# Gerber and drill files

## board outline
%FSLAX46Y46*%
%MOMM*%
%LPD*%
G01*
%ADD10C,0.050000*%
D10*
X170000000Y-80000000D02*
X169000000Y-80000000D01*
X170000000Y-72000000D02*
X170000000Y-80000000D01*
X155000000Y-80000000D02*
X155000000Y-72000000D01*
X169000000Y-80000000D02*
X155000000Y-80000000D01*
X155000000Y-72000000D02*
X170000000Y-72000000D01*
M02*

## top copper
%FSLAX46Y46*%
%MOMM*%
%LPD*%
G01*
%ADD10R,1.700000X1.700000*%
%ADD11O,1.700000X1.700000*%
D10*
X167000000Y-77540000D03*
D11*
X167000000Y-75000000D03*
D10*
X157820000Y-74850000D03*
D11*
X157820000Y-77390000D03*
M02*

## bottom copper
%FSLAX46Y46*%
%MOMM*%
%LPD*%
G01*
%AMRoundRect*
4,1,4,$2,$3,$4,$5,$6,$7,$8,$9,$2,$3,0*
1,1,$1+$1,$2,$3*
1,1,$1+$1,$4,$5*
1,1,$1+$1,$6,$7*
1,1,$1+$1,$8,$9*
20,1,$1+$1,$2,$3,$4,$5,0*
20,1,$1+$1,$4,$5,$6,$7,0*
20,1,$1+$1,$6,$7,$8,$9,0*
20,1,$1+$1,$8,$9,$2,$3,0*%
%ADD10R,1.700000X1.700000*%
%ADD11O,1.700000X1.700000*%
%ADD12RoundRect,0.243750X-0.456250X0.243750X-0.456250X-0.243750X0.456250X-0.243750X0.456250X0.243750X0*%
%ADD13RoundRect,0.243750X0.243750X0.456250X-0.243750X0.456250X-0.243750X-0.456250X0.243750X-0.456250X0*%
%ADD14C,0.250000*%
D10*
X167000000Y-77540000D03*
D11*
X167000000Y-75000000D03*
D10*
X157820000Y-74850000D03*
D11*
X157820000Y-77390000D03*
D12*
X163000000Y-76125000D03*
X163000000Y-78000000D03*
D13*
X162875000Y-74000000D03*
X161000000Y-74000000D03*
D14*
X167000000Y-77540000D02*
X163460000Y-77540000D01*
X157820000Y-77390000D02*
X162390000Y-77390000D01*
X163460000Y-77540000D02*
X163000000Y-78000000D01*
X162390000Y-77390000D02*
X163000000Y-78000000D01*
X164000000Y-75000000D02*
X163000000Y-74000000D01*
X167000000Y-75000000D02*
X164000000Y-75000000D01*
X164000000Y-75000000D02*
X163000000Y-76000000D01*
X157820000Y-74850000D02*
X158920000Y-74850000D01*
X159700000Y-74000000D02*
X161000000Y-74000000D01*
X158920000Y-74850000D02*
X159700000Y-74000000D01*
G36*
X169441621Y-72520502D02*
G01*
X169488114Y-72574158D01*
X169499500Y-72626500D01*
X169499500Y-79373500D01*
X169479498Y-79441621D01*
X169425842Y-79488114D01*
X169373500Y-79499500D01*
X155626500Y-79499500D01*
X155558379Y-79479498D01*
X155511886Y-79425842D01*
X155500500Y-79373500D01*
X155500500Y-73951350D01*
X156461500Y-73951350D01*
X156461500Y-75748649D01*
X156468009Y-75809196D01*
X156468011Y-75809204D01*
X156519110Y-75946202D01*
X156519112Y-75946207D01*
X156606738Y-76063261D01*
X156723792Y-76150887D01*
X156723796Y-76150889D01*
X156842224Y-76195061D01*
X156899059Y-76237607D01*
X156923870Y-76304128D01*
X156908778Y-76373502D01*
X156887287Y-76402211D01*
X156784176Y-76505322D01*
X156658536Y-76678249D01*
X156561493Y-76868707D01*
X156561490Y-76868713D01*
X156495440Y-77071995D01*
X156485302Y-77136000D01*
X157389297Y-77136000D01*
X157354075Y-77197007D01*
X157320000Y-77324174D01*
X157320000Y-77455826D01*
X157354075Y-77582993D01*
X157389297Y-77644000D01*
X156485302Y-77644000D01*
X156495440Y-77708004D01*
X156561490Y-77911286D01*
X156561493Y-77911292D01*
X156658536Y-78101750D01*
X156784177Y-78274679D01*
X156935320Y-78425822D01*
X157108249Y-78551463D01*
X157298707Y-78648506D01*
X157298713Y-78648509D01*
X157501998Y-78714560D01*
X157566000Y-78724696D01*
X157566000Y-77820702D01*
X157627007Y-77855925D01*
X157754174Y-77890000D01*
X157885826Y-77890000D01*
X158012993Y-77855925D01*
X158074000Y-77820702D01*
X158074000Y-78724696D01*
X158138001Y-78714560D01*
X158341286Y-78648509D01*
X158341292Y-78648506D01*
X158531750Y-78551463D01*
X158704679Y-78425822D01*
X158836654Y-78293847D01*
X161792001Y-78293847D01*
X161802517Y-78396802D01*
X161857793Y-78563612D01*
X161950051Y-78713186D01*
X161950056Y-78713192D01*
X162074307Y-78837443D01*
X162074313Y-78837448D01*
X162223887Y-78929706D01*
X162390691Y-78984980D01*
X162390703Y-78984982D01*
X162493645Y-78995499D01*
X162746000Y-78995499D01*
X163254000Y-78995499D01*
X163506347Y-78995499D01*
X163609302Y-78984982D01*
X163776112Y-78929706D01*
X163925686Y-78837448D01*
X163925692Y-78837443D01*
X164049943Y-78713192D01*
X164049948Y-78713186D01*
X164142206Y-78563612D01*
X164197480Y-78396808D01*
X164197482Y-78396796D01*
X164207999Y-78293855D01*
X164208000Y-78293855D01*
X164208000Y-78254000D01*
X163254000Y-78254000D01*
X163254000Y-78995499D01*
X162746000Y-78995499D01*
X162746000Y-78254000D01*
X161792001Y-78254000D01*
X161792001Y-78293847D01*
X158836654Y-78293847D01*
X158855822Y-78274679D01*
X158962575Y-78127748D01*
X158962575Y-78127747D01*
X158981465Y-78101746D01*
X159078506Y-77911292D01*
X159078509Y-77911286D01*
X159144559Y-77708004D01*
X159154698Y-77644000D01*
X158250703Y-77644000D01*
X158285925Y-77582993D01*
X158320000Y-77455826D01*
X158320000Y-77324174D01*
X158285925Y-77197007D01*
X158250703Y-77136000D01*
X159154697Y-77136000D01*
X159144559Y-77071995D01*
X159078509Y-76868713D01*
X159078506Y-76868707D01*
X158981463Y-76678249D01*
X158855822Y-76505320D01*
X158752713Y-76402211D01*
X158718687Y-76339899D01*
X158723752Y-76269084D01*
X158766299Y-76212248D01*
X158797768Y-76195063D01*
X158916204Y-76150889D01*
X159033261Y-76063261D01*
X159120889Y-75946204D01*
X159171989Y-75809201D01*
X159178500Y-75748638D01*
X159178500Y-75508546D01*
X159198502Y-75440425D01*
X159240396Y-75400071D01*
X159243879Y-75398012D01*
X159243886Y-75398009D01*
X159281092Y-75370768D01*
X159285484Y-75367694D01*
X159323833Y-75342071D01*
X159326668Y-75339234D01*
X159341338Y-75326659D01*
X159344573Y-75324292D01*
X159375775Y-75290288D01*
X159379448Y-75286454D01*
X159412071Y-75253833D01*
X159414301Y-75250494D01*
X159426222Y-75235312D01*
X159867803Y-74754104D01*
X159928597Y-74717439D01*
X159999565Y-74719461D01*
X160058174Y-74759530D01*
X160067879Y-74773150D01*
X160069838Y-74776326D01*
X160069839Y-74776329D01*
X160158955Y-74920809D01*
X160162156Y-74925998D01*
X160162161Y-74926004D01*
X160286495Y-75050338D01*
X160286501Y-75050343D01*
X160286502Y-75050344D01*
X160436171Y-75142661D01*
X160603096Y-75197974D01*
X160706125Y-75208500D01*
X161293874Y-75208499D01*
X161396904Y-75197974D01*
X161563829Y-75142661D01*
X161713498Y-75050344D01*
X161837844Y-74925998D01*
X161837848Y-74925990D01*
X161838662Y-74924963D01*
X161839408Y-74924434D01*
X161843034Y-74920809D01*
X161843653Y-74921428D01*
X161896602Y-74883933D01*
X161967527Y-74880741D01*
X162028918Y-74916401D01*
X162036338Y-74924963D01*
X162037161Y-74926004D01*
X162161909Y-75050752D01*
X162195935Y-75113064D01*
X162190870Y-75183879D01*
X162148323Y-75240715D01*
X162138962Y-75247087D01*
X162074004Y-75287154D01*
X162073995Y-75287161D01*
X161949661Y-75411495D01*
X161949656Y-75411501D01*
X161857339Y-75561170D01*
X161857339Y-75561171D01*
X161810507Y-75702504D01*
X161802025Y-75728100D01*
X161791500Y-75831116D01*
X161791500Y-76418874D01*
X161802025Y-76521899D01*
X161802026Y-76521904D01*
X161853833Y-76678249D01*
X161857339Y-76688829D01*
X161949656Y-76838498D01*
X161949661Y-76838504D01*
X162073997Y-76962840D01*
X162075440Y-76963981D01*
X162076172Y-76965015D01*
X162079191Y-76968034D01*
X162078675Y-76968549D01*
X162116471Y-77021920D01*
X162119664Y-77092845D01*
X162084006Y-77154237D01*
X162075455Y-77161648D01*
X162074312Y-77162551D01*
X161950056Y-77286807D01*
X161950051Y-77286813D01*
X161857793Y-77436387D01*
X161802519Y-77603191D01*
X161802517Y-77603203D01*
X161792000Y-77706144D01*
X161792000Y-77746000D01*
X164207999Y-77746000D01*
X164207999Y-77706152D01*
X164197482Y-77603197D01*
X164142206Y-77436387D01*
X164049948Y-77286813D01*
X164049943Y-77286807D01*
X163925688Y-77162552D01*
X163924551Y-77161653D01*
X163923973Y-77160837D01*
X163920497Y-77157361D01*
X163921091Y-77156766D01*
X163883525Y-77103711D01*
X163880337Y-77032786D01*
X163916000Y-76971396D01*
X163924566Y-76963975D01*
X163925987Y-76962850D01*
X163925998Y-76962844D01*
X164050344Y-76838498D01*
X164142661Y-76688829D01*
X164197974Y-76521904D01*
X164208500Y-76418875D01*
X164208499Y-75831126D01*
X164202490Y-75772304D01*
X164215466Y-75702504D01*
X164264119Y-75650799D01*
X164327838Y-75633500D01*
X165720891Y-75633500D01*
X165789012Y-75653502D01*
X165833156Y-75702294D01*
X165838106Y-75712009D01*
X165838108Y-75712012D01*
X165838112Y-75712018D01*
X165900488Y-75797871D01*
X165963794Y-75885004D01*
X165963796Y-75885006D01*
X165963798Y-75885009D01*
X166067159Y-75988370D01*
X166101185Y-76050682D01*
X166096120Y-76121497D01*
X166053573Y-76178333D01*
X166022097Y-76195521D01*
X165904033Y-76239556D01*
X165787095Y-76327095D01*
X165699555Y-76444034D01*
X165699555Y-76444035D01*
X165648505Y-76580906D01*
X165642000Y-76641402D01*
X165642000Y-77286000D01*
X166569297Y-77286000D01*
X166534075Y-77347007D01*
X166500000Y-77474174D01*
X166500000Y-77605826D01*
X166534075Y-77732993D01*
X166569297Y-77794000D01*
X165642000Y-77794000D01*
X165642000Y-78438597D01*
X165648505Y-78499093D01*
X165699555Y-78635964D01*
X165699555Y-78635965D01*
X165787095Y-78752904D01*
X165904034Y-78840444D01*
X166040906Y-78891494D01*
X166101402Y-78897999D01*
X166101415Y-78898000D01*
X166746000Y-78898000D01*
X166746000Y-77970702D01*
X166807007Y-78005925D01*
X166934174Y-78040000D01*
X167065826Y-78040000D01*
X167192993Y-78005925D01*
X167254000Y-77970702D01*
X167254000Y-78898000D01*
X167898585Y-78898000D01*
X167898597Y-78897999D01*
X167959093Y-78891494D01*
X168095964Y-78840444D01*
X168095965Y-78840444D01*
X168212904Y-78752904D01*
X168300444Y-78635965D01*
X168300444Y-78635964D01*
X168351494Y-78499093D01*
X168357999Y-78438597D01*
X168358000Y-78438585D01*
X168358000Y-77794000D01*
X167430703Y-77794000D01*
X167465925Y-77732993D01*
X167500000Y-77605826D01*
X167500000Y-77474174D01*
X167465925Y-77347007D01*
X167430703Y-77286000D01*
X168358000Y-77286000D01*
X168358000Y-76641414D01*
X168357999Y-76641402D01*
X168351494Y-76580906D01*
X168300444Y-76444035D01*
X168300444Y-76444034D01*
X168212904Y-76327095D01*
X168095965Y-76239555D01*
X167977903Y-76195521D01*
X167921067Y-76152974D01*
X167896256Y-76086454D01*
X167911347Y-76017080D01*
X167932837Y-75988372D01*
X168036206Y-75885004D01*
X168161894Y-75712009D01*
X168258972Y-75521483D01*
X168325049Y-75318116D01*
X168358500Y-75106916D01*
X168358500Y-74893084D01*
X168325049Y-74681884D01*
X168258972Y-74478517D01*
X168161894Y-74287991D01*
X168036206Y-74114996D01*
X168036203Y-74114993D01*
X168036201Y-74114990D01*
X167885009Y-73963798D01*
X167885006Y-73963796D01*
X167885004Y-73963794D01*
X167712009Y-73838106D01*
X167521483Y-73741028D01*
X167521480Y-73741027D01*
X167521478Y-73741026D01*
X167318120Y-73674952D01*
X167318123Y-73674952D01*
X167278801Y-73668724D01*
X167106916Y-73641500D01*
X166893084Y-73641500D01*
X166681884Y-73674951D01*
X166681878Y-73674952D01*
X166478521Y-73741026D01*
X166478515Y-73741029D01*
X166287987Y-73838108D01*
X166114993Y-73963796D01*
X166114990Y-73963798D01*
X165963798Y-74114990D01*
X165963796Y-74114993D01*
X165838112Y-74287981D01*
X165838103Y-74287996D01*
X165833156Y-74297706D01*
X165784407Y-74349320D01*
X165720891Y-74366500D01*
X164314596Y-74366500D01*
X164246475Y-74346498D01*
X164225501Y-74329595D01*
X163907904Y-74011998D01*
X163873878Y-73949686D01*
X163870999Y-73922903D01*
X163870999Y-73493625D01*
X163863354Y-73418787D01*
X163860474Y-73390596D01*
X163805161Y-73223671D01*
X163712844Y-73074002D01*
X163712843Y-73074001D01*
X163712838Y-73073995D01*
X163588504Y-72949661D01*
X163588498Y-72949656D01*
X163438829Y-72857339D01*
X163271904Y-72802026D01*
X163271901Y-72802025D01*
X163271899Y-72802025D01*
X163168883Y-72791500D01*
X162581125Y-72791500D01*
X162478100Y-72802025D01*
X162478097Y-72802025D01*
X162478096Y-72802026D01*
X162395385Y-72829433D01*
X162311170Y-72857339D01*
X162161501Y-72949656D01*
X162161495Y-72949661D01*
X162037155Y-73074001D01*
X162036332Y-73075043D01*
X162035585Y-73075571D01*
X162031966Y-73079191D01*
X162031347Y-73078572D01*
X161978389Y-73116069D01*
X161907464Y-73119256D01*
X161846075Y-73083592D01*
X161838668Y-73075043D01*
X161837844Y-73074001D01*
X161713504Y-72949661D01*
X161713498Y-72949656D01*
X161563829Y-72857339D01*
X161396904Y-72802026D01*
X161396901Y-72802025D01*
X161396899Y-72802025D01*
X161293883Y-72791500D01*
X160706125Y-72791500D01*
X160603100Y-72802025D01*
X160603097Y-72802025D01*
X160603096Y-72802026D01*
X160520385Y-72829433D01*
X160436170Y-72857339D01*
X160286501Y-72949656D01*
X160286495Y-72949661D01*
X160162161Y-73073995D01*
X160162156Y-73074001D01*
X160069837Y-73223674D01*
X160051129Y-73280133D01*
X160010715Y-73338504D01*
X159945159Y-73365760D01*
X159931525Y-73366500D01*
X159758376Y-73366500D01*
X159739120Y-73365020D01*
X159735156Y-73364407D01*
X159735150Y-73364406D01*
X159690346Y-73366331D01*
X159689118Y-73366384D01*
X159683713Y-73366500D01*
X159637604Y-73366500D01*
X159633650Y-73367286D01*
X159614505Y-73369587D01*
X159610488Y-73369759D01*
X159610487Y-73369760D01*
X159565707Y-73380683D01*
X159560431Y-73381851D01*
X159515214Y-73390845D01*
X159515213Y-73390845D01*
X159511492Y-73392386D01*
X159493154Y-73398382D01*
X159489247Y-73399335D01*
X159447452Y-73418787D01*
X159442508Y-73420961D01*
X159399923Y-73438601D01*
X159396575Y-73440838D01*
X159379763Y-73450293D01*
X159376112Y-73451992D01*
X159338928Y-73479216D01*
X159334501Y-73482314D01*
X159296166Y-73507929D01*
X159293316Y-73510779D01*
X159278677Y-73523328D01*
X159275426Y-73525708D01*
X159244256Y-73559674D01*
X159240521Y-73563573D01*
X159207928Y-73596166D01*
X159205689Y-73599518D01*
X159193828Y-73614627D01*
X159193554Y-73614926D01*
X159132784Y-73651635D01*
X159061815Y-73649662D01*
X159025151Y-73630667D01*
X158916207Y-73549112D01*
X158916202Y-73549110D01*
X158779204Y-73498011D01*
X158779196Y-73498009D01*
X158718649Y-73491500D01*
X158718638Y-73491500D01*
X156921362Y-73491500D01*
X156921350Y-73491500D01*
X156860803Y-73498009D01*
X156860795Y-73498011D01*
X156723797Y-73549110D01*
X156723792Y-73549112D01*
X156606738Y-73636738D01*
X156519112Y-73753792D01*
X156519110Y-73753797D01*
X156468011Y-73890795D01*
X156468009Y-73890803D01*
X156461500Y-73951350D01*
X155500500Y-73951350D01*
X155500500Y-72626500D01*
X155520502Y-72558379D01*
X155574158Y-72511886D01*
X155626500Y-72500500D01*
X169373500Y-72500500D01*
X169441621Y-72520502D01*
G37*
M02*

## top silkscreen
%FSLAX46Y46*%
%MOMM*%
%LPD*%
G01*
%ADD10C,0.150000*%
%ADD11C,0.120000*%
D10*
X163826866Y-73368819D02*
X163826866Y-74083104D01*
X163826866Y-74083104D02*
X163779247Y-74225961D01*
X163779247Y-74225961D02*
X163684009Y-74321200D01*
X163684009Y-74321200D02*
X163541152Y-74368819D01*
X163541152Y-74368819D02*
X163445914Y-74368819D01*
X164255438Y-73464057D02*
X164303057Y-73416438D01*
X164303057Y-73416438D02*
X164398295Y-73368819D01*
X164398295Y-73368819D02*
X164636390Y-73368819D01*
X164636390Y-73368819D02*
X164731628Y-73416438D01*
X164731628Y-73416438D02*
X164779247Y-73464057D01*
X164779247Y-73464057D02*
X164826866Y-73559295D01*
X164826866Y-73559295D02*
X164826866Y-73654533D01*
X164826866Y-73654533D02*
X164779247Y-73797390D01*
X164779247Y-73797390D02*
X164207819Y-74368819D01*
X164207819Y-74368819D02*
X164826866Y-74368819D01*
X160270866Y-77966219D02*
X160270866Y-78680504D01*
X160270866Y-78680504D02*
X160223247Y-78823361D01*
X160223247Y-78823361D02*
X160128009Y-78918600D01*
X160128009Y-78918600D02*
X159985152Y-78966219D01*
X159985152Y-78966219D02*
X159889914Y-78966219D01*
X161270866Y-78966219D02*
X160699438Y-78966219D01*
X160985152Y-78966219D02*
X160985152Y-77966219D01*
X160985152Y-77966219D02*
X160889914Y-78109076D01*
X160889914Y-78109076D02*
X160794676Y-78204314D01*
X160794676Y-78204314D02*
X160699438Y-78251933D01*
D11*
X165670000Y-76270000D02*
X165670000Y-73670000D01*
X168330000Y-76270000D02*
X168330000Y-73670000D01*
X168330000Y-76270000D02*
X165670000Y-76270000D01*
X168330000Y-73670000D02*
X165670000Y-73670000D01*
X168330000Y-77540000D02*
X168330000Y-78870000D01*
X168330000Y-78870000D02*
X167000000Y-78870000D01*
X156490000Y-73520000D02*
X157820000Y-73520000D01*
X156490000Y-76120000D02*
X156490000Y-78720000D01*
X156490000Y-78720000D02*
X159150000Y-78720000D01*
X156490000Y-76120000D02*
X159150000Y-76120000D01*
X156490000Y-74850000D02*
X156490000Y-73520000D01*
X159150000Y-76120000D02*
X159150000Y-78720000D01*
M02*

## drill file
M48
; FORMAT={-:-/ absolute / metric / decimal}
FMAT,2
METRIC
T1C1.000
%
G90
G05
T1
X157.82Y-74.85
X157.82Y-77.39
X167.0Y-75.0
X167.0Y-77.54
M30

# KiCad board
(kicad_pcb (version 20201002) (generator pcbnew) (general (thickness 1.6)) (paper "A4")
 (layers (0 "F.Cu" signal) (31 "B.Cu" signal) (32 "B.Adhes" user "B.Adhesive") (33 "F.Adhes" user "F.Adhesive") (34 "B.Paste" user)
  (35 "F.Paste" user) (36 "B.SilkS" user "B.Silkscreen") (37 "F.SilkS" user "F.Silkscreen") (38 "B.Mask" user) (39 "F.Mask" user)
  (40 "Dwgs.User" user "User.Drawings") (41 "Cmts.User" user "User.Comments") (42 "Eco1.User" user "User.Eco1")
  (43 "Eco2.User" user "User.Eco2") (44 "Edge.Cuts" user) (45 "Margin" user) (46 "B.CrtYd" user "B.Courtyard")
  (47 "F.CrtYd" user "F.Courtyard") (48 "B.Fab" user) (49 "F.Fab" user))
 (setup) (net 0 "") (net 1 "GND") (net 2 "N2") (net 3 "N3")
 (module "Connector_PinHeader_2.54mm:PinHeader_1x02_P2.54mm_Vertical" (layer "F.Cu") (at 167 77.54 180)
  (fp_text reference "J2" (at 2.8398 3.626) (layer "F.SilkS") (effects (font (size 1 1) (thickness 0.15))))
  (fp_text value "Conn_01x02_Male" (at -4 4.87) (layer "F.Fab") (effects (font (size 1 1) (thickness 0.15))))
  (fp_line (start 1.33 1.27) (end 1.33 3.87) (layer "F.SilkS") (width 0.12))
  (fp_line (start -1.33 1.27) (end -1.33 3.87) (layer "F.SilkS") (width 0.12))
  (fp_line (start -1.33 1.27) (end 1.33 1.27) (layer "F.SilkS") (width 0.12))
  (fp_line (start -1.33 3.87) (end 1.33 3.87) (layer "F.SilkS") (width 0.12))
  (fp_line (start -1.33 0) (end -1.33 -1.33) (layer "F.SilkS") (width 0.12))
  (fp_line (start -1.33 -1.33) (end 0 -1.33) (layer "F.SilkS") (width 0.12))
  (pad "1" thru_hole rect (at 0 0 180) (size 1.7 1.7) (drill 1) (layers *.Cu *.Mask) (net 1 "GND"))
  (pad "2" thru_hole oval (at 0 2.54 180) (size 1.7 1.7) (drill 1) (layers *.Cu *.Mask) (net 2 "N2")))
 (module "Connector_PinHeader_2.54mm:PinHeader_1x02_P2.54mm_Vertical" (layer "F.Cu") (at 157.82 74.85)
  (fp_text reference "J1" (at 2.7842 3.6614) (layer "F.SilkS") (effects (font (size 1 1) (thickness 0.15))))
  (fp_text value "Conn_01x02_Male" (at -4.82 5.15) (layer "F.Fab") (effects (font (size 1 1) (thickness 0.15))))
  (fp_line (start -1.33 -1.33) (end 0 -1.33) (layer "F.SilkS") (width 0.12))
  (fp_line (start -1.33 1.27) (end -1.33 3.87) (layer "F.SilkS") (width 0.12))
  (fp_line (start -1.33 3.87) (end 1.33 3.87) (layer "F.SilkS") (width 0.12))
  (fp_line (start -1.33 1.27) (end 1.33 1.27) (layer "F.SilkS") (width 0.12))
  (fp_line (start -1.33 0) (end -1.33 -1.33) (layer "F.SilkS") (width 0.12))
  (fp_line (start 1.33 1.27) (end 1.33 3.87) (layer "F.SilkS") (width 0.12))
  (pad "1" thru_hole rect (at 0 0) (size 1.7 1.7) (drill 1) (layers *.Cu *.Mask) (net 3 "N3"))
  (pad "2" thru_hole oval (at 0 2.54) (size 1.7 1.7) (drill 1) (layers *.Cu *.Mask) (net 1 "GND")))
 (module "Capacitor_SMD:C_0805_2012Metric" (layer "B.Cu") (at 163 77.0625 -90)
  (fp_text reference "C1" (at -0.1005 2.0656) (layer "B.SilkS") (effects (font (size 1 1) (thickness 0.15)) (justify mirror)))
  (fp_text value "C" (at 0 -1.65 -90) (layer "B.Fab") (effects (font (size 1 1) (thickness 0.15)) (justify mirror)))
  (pad "1" smd roundrect (at -0.9375 0 270) (size 0.975 1.4) (layers "B.Cu" "B.Paste" "B.Mask") (roundrect_rratio 0.25) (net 2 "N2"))
  (pad "2" smd roundrect (at 0.9375 0 270) (size 0.975 1.4) (layers "B.Cu" "B.Paste" "B.Mask") (roundrect_rratio 0.25) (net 1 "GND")))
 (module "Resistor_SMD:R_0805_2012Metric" (layer "B.Cu") (at 161.9375 74 180)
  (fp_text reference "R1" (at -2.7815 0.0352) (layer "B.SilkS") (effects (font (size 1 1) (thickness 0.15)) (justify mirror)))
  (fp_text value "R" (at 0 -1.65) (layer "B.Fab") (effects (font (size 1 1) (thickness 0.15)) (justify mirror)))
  (pad "1" smd roundrect (at -0.9375 0 180) (size 0.975 1.4) (layers "B.Cu" "B.Paste" "B.Mask") (roundrect_rratio 0.25) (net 2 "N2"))
  (pad "2" smd roundrect (at 0.9375 0 180) (size 0.975 1.4) (layers "B.Cu" "B.Paste" "B.Mask") (roundrect_rratio 0.25) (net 3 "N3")))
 (gr_line (start 170 80) (end 169 80) (layer "Edge.Cuts") (width 0.05))
 (gr_line (start 170 72) (end 170 80) (layer "Edge.Cuts") (width 0.05))
 (gr_line (start 155 80) (end 155 72) (layer "Edge.Cuts") (width 0.05))
 (gr_line (start 169 80) (end 155 80) (layer "Edge.Cuts") (width 0.05))
 (gr_line (start 155 72) (end 170 72) (layer "Edge.Cuts") (width 0.05))
 (segment (start 167 77.54) (end 163.46 77.54) (width 0.25) (layer "B.Cu") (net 1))
 (segment (start 157.82 77.39) (end 162.39 77.39) (width 0.25) (layer "B.Cu") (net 1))
 (segment (start 163.46 77.54) (end 163 78) (width 0.25) (layer "B.Cu") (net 1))
 (segment (start 162.39 77.39) (end 163 78) (width 0.25) (layer "B.Cu") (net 1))
 (segment (start 164 75) (end 163 74) (width 0.25) (layer "B.Cu") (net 2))
 (segment (start 167 75) (end 164 75) (width 0.25) (layer "B.Cu") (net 2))
 (segment (start 164 75) (end 163 76) (width 0.25) (layer "B.Cu") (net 2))
 (segment (start 157.82 74.85) (end 158.92 74.85) (width 0.25) (layer "B.Cu") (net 3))
 (segment (start 159.7 74) (end 161 74) (width 0.25) (layer "B.Cu") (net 3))
 (segment (start 158.92 74.85) (end 159.7 74) (width 0.25) (layer "B.Cu") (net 3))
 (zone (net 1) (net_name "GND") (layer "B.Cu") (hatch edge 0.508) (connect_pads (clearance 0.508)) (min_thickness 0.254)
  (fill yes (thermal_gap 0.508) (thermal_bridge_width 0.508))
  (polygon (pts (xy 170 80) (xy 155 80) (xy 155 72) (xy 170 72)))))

